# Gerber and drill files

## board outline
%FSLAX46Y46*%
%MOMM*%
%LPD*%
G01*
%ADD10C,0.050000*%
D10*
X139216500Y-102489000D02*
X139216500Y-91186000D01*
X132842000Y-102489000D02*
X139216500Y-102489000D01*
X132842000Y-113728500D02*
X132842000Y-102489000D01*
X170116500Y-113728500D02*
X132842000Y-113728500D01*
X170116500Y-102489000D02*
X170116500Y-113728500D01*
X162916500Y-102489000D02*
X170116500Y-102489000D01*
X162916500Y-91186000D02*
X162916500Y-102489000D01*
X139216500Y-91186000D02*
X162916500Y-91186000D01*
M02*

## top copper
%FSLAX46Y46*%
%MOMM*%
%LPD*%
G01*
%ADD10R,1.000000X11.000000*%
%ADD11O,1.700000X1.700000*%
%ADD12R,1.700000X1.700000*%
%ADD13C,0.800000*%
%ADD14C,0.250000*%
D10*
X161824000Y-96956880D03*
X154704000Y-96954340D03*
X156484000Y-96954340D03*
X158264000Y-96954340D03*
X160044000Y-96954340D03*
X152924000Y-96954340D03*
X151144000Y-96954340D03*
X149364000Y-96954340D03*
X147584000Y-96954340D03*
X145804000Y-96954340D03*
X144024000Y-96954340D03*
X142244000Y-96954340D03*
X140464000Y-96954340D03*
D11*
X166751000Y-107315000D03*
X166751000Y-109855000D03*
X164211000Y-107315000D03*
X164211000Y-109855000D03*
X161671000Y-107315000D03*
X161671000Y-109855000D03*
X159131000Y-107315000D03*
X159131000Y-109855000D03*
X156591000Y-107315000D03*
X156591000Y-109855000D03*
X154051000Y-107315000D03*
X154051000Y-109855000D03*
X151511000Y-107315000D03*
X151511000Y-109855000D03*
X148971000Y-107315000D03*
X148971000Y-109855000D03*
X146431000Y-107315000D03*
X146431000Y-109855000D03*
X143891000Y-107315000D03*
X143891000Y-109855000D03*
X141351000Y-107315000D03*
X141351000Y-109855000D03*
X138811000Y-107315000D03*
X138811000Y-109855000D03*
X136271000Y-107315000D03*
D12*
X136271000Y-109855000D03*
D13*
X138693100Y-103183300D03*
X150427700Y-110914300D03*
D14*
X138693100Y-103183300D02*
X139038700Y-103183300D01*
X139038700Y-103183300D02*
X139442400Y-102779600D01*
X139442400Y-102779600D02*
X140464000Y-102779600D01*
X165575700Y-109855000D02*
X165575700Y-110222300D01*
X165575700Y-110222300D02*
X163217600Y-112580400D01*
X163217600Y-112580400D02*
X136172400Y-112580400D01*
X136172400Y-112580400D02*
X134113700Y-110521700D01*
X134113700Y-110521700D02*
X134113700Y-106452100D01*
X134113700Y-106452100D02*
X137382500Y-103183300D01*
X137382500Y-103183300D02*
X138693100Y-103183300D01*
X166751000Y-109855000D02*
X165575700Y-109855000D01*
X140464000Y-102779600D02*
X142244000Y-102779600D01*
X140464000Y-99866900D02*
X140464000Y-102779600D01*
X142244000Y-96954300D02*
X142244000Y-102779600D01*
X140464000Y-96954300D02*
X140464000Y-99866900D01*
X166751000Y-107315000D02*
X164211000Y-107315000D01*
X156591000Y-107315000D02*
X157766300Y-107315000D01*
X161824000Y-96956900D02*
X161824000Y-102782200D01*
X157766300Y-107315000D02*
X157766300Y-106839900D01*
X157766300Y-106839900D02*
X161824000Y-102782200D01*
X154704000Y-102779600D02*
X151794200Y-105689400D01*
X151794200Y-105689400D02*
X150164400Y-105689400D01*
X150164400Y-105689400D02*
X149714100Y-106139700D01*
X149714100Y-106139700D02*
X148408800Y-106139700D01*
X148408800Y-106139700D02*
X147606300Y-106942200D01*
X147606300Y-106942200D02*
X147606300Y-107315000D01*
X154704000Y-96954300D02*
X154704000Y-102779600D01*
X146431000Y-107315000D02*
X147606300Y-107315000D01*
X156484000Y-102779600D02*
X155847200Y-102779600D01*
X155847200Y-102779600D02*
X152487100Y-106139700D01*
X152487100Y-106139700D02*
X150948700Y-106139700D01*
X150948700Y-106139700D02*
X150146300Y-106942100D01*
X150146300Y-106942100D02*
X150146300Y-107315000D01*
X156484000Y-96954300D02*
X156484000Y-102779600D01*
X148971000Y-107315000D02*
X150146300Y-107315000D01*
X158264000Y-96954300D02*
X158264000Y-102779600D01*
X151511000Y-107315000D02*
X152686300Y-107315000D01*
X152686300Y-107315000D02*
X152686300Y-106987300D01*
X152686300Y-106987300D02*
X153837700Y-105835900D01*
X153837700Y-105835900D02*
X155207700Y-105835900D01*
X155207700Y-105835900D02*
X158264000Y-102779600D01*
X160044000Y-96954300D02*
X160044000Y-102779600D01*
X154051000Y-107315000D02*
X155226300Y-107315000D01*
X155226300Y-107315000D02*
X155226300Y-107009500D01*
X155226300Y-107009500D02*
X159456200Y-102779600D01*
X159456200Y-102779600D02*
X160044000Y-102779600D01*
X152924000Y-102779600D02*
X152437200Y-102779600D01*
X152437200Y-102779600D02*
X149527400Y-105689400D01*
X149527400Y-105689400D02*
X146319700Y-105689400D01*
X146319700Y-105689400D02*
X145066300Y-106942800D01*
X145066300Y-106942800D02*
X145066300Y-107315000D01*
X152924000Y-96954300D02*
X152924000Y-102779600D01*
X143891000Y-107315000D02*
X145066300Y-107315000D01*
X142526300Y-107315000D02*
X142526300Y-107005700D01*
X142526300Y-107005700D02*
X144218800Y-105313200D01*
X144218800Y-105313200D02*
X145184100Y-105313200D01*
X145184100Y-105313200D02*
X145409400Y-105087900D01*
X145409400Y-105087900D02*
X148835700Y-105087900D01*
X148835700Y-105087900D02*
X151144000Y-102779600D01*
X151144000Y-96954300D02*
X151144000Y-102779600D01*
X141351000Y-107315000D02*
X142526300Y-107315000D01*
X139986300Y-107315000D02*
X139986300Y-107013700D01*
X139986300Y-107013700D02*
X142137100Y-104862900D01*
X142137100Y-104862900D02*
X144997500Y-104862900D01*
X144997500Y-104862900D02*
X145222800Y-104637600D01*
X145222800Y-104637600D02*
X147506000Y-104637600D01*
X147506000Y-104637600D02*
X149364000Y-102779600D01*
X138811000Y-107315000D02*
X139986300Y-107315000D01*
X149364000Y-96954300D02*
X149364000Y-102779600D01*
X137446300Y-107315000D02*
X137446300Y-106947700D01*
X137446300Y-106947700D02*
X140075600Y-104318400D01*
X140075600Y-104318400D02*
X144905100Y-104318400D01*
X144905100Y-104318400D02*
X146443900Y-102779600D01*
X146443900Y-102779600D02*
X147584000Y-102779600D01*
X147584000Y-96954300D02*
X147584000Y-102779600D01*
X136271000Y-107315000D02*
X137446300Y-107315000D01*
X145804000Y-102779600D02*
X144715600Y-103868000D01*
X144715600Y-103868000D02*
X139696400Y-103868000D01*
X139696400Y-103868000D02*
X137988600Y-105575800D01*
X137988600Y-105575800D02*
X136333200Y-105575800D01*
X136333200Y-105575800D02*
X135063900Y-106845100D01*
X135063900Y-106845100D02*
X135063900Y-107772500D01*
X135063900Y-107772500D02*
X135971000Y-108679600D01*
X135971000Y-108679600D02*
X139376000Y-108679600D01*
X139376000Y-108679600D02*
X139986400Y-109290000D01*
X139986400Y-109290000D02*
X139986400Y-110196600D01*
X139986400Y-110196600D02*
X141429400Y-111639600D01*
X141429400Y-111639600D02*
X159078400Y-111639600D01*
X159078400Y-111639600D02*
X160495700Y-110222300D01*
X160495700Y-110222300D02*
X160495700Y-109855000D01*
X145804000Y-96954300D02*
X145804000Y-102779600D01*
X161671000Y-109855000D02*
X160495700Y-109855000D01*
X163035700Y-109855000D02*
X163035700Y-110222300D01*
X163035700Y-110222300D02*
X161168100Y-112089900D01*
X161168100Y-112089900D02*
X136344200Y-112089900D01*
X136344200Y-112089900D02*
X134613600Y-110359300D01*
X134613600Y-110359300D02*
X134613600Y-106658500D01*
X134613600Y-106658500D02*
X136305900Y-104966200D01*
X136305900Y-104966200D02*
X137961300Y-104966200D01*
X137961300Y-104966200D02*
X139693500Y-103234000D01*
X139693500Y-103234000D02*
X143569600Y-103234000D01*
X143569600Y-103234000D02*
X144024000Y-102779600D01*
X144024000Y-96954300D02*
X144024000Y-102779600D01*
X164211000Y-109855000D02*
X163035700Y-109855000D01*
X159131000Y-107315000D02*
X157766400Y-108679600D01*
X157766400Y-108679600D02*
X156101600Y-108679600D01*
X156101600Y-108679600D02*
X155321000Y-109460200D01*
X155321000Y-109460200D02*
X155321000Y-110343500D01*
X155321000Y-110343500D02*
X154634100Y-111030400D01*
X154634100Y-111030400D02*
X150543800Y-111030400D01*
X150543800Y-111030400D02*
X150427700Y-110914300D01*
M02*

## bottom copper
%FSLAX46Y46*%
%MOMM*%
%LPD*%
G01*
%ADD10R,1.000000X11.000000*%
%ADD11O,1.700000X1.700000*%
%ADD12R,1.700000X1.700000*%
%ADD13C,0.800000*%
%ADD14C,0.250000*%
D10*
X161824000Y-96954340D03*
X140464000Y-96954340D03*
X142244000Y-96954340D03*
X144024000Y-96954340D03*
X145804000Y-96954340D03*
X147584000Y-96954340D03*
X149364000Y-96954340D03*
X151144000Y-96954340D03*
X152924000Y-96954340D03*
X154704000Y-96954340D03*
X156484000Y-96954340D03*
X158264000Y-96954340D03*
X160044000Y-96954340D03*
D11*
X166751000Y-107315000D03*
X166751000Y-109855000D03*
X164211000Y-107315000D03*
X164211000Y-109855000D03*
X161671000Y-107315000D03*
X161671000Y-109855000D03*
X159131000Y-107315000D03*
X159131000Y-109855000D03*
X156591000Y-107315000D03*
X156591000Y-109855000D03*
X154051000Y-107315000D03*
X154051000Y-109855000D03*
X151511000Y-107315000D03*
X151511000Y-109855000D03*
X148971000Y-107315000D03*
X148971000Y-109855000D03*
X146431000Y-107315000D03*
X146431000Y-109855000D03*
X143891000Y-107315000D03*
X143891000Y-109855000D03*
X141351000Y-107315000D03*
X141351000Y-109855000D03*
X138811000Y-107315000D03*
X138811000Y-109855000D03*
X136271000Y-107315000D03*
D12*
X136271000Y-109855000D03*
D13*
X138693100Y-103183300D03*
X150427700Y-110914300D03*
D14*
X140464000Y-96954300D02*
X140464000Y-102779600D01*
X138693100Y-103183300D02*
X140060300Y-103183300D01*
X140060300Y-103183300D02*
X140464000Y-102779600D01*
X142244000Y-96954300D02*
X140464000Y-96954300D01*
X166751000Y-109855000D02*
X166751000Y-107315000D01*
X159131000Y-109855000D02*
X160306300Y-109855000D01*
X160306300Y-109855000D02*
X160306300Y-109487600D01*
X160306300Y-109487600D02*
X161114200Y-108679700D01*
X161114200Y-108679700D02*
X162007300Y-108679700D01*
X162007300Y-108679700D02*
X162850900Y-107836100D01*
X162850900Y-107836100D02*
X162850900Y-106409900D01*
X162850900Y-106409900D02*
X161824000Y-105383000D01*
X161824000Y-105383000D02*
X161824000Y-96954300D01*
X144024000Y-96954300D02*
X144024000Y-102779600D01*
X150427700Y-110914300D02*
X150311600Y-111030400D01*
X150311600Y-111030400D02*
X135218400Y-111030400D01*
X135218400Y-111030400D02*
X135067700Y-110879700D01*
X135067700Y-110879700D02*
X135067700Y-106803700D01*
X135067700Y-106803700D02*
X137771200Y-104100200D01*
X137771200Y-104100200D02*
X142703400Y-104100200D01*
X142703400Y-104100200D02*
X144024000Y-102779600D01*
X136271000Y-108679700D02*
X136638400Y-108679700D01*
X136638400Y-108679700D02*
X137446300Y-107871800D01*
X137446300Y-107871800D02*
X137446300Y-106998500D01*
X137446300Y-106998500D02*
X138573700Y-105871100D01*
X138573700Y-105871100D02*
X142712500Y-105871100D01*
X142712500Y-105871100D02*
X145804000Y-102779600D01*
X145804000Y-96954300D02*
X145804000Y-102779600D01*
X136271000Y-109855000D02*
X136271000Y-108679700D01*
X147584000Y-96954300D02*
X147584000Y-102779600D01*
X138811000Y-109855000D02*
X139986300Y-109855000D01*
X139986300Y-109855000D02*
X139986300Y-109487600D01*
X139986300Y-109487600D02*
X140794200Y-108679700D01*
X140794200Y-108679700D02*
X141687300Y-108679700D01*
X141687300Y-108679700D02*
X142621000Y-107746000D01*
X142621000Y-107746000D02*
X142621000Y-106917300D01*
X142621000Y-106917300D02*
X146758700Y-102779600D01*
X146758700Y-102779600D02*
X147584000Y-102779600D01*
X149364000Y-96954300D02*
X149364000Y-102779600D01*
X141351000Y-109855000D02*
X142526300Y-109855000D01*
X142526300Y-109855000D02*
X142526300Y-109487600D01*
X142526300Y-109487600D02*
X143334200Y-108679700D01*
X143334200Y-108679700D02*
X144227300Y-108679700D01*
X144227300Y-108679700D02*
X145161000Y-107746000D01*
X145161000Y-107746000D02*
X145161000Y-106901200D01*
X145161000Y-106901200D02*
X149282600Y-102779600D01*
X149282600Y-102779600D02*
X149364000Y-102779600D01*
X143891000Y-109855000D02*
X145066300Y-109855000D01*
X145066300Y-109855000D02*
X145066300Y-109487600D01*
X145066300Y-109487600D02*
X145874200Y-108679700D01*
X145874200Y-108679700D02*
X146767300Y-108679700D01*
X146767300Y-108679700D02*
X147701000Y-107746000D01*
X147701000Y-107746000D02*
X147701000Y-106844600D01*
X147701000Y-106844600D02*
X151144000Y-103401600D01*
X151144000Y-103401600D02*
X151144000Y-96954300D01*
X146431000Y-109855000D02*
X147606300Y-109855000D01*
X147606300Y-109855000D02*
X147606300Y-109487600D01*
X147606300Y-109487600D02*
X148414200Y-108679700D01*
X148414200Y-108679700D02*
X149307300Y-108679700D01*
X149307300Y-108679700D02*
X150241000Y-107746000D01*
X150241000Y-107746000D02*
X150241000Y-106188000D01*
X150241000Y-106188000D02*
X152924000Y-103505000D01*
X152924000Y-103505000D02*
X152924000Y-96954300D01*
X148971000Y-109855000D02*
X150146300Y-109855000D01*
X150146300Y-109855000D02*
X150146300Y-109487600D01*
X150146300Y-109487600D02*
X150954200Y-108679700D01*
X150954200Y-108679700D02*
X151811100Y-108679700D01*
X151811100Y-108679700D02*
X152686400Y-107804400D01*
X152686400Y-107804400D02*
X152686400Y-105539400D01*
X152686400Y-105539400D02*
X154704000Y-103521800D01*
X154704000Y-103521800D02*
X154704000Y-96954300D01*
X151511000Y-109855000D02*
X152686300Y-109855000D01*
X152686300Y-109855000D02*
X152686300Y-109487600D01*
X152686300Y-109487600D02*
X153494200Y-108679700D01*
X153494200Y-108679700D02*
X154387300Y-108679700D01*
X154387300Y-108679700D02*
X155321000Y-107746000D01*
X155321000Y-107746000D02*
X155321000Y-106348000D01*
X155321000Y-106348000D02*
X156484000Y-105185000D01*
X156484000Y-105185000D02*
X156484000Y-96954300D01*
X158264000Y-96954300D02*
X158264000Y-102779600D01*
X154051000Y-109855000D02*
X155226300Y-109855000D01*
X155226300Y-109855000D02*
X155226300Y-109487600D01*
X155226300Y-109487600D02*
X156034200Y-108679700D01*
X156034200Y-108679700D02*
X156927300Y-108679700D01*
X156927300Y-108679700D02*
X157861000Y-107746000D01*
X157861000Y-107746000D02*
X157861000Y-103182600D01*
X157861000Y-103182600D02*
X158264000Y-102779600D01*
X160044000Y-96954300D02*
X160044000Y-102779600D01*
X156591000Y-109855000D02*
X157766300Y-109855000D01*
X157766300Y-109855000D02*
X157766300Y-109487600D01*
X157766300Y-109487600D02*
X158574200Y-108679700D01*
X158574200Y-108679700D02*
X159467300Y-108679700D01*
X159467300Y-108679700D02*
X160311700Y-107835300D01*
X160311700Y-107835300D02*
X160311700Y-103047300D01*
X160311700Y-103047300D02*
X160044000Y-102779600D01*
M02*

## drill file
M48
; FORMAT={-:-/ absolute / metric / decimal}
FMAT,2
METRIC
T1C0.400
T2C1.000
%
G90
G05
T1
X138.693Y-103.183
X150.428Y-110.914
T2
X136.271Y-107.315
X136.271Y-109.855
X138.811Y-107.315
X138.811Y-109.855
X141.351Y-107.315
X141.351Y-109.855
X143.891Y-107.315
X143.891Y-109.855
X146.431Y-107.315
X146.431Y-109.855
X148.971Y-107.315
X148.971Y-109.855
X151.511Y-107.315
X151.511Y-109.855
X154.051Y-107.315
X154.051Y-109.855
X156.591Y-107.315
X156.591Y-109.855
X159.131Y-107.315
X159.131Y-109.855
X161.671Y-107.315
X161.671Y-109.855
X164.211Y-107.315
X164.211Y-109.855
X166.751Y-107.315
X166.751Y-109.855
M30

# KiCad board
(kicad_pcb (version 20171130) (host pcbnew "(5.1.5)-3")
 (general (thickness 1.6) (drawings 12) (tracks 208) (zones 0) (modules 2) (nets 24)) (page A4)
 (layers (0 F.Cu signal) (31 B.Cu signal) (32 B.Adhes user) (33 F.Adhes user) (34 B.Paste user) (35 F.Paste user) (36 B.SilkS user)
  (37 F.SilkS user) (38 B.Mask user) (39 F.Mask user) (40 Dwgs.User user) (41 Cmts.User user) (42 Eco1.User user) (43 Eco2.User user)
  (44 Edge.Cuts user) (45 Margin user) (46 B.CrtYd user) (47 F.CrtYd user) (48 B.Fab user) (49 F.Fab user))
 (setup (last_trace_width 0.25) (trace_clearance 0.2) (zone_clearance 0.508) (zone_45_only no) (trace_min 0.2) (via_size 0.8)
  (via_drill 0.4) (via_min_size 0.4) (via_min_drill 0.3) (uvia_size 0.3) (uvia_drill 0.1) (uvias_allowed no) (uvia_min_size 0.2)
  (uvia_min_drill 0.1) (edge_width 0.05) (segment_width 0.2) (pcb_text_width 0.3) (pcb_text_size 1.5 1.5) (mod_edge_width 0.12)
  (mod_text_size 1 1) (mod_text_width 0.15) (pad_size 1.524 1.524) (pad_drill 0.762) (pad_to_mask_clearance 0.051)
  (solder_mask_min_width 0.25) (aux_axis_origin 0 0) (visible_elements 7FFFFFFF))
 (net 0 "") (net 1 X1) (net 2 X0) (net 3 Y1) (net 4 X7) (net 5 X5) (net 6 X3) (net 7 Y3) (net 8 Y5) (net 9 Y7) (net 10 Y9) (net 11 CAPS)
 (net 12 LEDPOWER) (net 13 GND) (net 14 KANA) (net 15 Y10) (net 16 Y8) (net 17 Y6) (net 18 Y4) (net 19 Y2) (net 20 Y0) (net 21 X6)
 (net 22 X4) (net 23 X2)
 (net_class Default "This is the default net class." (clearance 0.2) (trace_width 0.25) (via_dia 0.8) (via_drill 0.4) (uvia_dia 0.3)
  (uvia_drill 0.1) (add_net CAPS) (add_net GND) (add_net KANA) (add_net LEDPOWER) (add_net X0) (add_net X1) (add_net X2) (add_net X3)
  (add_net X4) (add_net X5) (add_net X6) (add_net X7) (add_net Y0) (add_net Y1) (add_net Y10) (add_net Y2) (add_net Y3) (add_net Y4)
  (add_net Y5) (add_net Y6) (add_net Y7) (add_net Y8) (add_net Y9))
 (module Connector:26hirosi (layer F.Cu) (at 152.464 97.028)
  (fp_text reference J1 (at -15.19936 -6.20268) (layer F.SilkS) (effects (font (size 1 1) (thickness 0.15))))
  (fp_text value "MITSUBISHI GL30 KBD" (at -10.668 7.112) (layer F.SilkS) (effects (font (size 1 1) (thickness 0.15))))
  (pad 25 connect rect (at 9.36 -0.07112) (size 1 11) (layers F.Cu F.Mask) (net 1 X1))
  (pad 26 connect rect (at 9.36 -0.07366) (size 1 11) (layers B.Cu B.Mask) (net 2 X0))
  (pad 17 connect rect (at 2.24 -0.07366) (size 1 11) (layers F.Cu F.Mask) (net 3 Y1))
  (pad 19 connect rect (at 4.02 -0.07366) (size 1 11) (layers F.Cu F.Mask) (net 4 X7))
  (pad 21 connect rect (at 5.8 -0.07366) (size 1 11) (layers F.Cu F.Mask) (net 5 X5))
  (pad 23 connect rect (at 7.58 -0.07366) (size 1 11) (layers F.Cu F.Mask) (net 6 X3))
  (pad 15 connect rect (at 0.46 -0.07366) (size 1 11) (layers F.Cu F.Mask) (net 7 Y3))
  (pad 13 connect rect (at -1.32 -0.07366) (size 1 11) (layers F.Cu F.Mask) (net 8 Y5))
  (pad 11 connect rect (at -3.1 -0.07366) (size 1 11) (layers F.Cu F.Mask) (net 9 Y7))
  (pad 9 connect rect (at -4.88 -0.07366) (size 1 11) (layers F.Cu F.Mask) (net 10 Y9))
  (pad 7 connect rect (at -6.66 -0.07366) (size 1 11) (layers F.Cu F.Mask) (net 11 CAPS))
  (pad 5 connect rect (at -8.44 -0.07366) (size 1 11) (layers F.Cu F.Mask) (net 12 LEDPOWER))
  (pad 3 connect rect (at -10.22 -0.07366) (size 1 11) (layers F.Cu F.Mask) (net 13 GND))
  (pad 1 connect rect (at -12 -0.07366) (size 1 11) (layers F.Cu F.Mask) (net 13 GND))
  (pad 2 connect rect (at -12 -0.07366) (size 1 11) (layers B.Cu B.Mask) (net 13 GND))
  (pad 4 connect rect (at -10.22 -0.07366) (size 1 11) (layers B.Cu B.Mask) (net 13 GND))
  (pad 6 connect rect (at -8.44 -0.07366) (size 1 11) (layers B.Cu B.Mask) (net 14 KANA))
  (pad 8 connect rect (at -6.66 -0.07366) (size 1 11) (layers B.Cu B.Mask) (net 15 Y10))
  (pad 10 connect rect (at -4.88 -0.07366) (size 1 11) (layers B.Cu B.Mask) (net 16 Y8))
  (pad 12 connect rect (at -3.1 -0.07366) (size 1 11) (layers B.Cu B.Mask) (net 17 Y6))
  (pad 14 connect rect (at -1.32 -0.07366) (size 1 11) (layers B.Cu B.Mask) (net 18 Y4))
  (pad 16 connect rect (at 0.46 -0.07366) (size 1 11) (layers B.Cu B.Mask) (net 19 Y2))
  (pad 18 connect rect (at 2.24 -0.07366) (size 1 11) (layers B.Cu B.Mask) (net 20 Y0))
  (pad 20 connect rect (at 4.02 -0.07366) (size 1 11) (layers B.Cu B.Mask) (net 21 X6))
  (pad 22 connect rect (at 5.8 -0.07366) (size 1 11) (layers B.Cu B.Mask) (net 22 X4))
  (pad 24 connect rect (at 7.58 -0.07366) (size 1 11) (layers B.Cu B.Mask) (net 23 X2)))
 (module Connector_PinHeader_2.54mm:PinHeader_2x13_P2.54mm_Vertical (layer F.Cu) (at 136.271 109.855 90)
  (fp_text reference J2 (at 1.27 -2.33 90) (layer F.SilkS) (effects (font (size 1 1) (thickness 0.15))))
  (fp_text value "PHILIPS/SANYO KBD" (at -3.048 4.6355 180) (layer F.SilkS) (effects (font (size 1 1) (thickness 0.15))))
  (pad 26 thru_hole oval (at 2.54 30.48 90) (size 1.7 1.7) (drill 1) (layers *.Cu *.Mask) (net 13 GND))
  (pad 25 thru_hole oval (at 0 30.48 90) (size 1.7 1.7) (drill 1) (layers *.Cu *.Mask) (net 13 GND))
  (pad 24 thru_hole oval (at 2.54 27.94 90) (size 1.7 1.7) (drill 1) (layers *.Cu *.Mask) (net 13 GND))
  (pad 23 thru_hole oval (at 0 27.94 90) (size 1.7 1.7) (drill 1) (layers *.Cu *.Mask) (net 12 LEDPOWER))
  (pad 22 thru_hole oval (at 2.54 25.4 90) (size 1.7 1.7) (drill 1) (layers *.Cu *.Mask))
  (pad 21 thru_hole oval (at 0 25.4 90) (size 1.7 1.7) (drill 1) (layers *.Cu *.Mask) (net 11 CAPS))
  (pad 20 thru_hole oval (at 2.54 22.86 90) (size 1.7 1.7) (drill 1) (layers *.Cu *.Mask) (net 14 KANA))
  (pad 19 thru_hole oval (at 0 22.86 90) (size 1.7 1.7) (drill 1) (layers *.Cu *.Mask) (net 2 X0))
  (pad 18 thru_hole oval (at 2.54 20.32 90) (size 1.7 1.7) (drill 1) (layers *.Cu *.Mask) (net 1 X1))
  (pad 17 thru_hole oval (at 0 20.32 90) (size 1.7 1.7) (drill 1) (layers *.Cu *.Mask) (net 23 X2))
  (pad 16 thru_hole oval (at 2.54 17.78 90) (size 1.7 1.7) (drill 1) (layers *.Cu *.Mask) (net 6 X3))
  (pad 15 thru_hole oval (at 0 17.78 90) (size 1.7 1.7) (drill 1) (layers *.Cu *.Mask) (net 22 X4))
  (pad 14 thru_hole oval (at 2.54 15.24 90) (size 1.7 1.7) (drill 1) (layers *.Cu *.Mask) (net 5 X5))
  (pad 13 thru_hole oval (at 0 15.24 90) (size 1.7 1.7) (drill 1) (layers *.Cu *.Mask) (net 21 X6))
  (pad 12 thru_hole oval (at 2.54 12.7 90) (size 1.7 1.7) (drill 1) (layers *.Cu *.Mask) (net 4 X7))
  (pad 11 thru_hole oval (at 0 12.7 90) (size 1.7 1.7) (drill 1) (layers *.Cu *.Mask) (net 20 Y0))
  (pad 10 thru_hole oval (at 2.54 10.16 90) (size 1.7 1.7) (drill 1) (layers *.Cu *.Mask) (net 3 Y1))
  (pad 9 thru_hole oval (at 0 10.16 90) (size 1.7 1.7) (drill 1) (layers *.Cu *.Mask) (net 19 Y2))
  (pad 8 thru_hole oval (at 2.54 7.62 90) (size 1.7 1.7) (drill 1) (layers *.Cu *.Mask) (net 7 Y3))
  (pad 7 thru_hole oval (at 0 7.62 90) (size 1.7 1.7) (drill 1) (layers *.Cu *.Mask) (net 18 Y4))
  (pad 6 thru_hole oval (at 2.54 5.08 90) (size 1.7 1.7) (drill 1) (layers *.Cu *.Mask) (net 8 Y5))
  (pad 5 thru_hole oval (at 0 5.08 90) (size 1.7 1.7) (drill 1) (layers *.Cu *.Mask) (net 17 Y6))
  (pad 4 thru_hole oval (at 2.54 2.54 90) (size 1.7 1.7) (drill 1) (layers *.Cu *.Mask) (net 9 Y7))
  (pad 3 thru_hole oval (at 0 2.54 90) (size 1.7 1.7) (drill 1) (layers *.Cu *.Mask) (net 16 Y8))
  (pad 2 thru_hole oval (at 2.54 0 90) (size 1.7 1.7) (drill 1) (layers *.Cu *.Mask) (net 10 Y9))
  (pad 1 thru_hole rect (at 0 0 90) (size 1.7 1.7) (drill 1) (layers *.Cu *.Mask) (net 15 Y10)))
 (gr_line (start 139.2165 102.489) (end 139.2165 91.186) (layer Edge.Cuts) (width 0.05))
 (gr_line (start 132.842 102.489) (end 139.2165 102.489) (layer Edge.Cuts) (width 0.05))
 (gr_line (start 132.842 113.7285) (end 132.842 102.489) (layer Edge.Cuts) (width 0.05))
 (gr_line (start 170.1165 113.7285) (end 132.842 113.7285) (layer Edge.Cuts) (width 0.05))
 (gr_line (start 170.1165 102.489) (end 170.1165 113.7285) (layer Edge.Cuts) (width 0.05))
 (gr_line (start 162.9165 102.489) (end 170.1165 102.489) (layer Edge.Cuts) (width 0.05))
 (gr_line (start 162.9165 91.186) (end 162.9165 102.489) (layer Edge.Cuts) (width 0.05))
 (gr_line (start 139.2165 91.186) (end 162.9165 91.186) (layer Edge.Cuts) (width 0.05))
 (segment (start 138.6931 103.1833) (end 139.0387 103.1833) (width 0.25) (layer F.Cu) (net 13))
 (segment (start 139.0387 103.1833) (end 139.4424 102.7796) (width 0.25) (layer F.Cu) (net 13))
 (segment (start 139.4424 102.7796) (end 140.464 102.7796) (width 0.25) (layer F.Cu) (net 13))
 (segment (start 165.5757 109.855) (end 165.5757 110.2223) (width 0.25) (layer F.Cu) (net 13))
 (segment (start 165.5757 110.2223) (end 163.2176 112.5804) (width 0.25) (layer F.Cu) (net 13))
 (segment (start 163.2176 112.5804) (end 136.1724 112.5804) (width 0.25) (layer F.Cu) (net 13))
 (segment (start 136.1724 112.5804) (end 134.1137 110.5217) (width 0.25) (layer F.Cu) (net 13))
 (segment (start 134.1137 110.5217) (end 134.1137 106.4521) (width 0.25) (layer F.Cu) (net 13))
 (segment (start 134.1137 106.4521) (end 137.3825 103.1833) (width 0.25) (layer F.Cu) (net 13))
 (segment (start 137.3825 103.1833) (end 138.6931 103.1833) (width 0.25) (layer F.Cu) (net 13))
 (segment (start 140.464 96.9543) (end 140.464 102.7796) (width 0.25) (layer B.Cu) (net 13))
 (segment (start 138.6931 103.1833) (end 140.0603 103.1833) (width 0.25) (layer B.Cu) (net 13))
 (segment (start 140.0603 103.1833) (end 140.464 102.7796) (width 0.25) (layer B.Cu) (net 13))
 (segment (start 142.244 96.9543) (end 140.464 96.9543) (width 0.25) (layer B.Cu) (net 13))
 (segment (start 166.751 109.855) (end 165.5757 109.855) (width 0.25) (layer F.Cu) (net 13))
 (segment (start 140.464 102.7796) (end 142.244 102.7796) (width 0.25) (layer F.Cu) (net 13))
 (segment (start 140.464 99.8669) (end 140.464 102.7796) (width 0.25) (layer F.Cu) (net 13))
 (segment (start 166.751 109.855) (end 166.751 107.315) (width 0.25) (layer B.Cu) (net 13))
 (segment (start 142.244 96.9543) (end 142.244 102.7796) (width 0.25) (layer F.Cu) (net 13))
 (segment (start 140.464 96.9543) (end 140.464 99.8669) (width 0.25) (layer F.Cu) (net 13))
 (segment (start 166.751 107.315) (end 164.211 107.315) (width 0.25) (layer F.Cu) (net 13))
 (via (at 138.6931 103.1833) (size 0.8) (layers F.Cu B.Cu) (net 13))
 (segment (start 156.591 107.315) (end 157.7663 107.315) (width 0.25) (layer F.Cu) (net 1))
 (segment (start 161.824 96.9569) (end 161.824 102.7822) (width 0.25) (layer F.Cu) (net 1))
 (segment (start 157.7663 107.315) (end 157.7663 106.8399) (width 0.25) (layer F.Cu) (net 1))
 (segment (start 157.7663 106.8399) (end 161.824 102.7822) (width 0.25) (layer F.Cu) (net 1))
 (segment (start 159.131 109.855) (end 160.3063 109.855) (width 0.25) (layer B.Cu) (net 2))
 (segment (start 160.3063 109.855) (end 160.3063 109.4876) (width 0.25) (layer B.Cu) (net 2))
 (segment (start 160.3063 109.4876) (end 161.1142 108.6797) (width 0.25) (layer B.Cu) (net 2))
 (segment (start 161.1142 108.6797) (end 162.0073 108.6797) (width 0.25) (layer B.Cu) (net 2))
 (segment (start 162.0073 108.6797) (end 162.8509 107.8361) (width 0.25) (layer B.Cu) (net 2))
 (segment (start 162.8509 107.8361) (end 162.8509 106.4099) (width 0.25) (layer B.Cu) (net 2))
 (segment (start 162.8509 106.4099) (end 161.824 105.383) (width 0.25) (layer B.Cu) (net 2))
 (segment (start 161.824 105.383) (end 161.824 96.9543) (width 0.25) (layer B.Cu) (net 2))
 (segment (start 154.704 102.7796) (end 151.7942 105.6894) (width 0.25) (layer F.Cu) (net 3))
 (segment (start 151.7942 105.6894) (end 150.1644 105.6894) (width 0.25) (layer F.Cu) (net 3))
 (segment (start 150.1644 105.6894) (end 149.7141 106.1397) (width 0.25) (layer F.Cu) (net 3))
 (segment (start 149.7141 106.1397) (end 148.4088 106.1397) (width 0.25) (layer F.Cu) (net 3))
 (segment (start 148.4088 106.1397) (end 147.6063 106.9422) (width 0.25) (layer F.Cu) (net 3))
 (segment (start 147.6063 106.9422) (end 147.6063 107.315) (width 0.25) (layer F.Cu) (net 3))
 (segment (start 154.704 96.9543) (end 154.704 102.7796) (width 0.25) (layer F.Cu) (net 3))
 (segment (start 146.431 107.315) (end 147.6063 107.315) (width 0.25) (layer F.Cu) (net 3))
 (segment (start 156.484 102.7796) (end 155.8472 102.7796) (width 0.25) (layer F.Cu) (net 4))
 (segment (start 155.8472 102.7796) (end 152.4871 106.1397) (width 0.25) (layer F.Cu) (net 4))
 (segment (start 152.4871 106.1397) (end 150.9487 106.1397) (width 0.25) (layer F.Cu) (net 4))
 (segment (start 150.9487 106.1397) (end 150.1463 106.9421) (width 0.25) (layer F.Cu) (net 4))
 (segment (start 150.1463 106.9421) (end 150.1463 107.315) (width 0.25) (layer F.Cu) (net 4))
 (segment (start 156.484 96.9543) (end 156.484 102.7796) (width 0.25) (layer F.Cu) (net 4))
 (segment (start 148.971 107.315) (end 150.1463 107.315) (width 0.25) (layer F.Cu) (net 4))
 (segment (start 158.264 96.9543) (end 158.264 102.7796) (width 0.25) (layer F.Cu) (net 5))
 (segment (start 151.511 107.315) (end 152.6863 107.315) (width 0.25) (layer F.Cu) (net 5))
 (segment (start 152.6863 107.315) (end 152.6863 106.9873) (width 0.25) (layer F.Cu) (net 5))
 (segment (start 152.6863 106.9873) (end 153.8377 105.8359) (width 0.25) (layer F.Cu) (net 5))
 (segment (start 153.8377 105.8359) (end 155.2077 105.8359) (width 0.25) (layer F.Cu) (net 5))
 (segment (start 155.2077 105.8359) (end 158.264 102.7796) (width 0.25) (layer F.Cu) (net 5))
 (segment (start 160.044 96.9543) (end 160.044 102.7796) (width 0.25) (layer F.Cu) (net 6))
 (segment (start 154.051 107.315) (end 155.2263 107.315) (width 0.25) (layer F.Cu) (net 6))
 (segment (start 155.2263 107.315) (end 155.2263 107.0095) (width 0.25) (layer F.Cu) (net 6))
 (segment (start 155.2263 107.0095) (end 159.4562 102.7796) (width 0.25) (layer F.Cu) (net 6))
 (segment (start 159.4562 102.7796) (end 160.044 102.7796) (width 0.25) (layer F.Cu) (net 6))
 (segment (start 152.924 102.7796) (end 152.4372 102.7796) (width 0.25) (layer F.Cu) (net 7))
 (segment (start 152.4372 102.7796) (end 149.5274 105.6894) (width 0.25) (layer F.Cu) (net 7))
 (segment (start 149.5274 105.6894) (end 146.3197 105.6894) (width 0.25) (layer F.Cu) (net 7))
 (segment (start 146.3197 105.6894) (end 145.0663 106.9428) (width 0.25) (layer F.Cu) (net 7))
 (segment (start 145.0663 106.9428) (end 145.0663 107.315) (width 0.25) (layer F.Cu) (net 7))
 (segment (start 152.924 96.9543) (end 152.924 102.7796) (width 0.25) (layer F.Cu) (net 7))
 (segment (start 143.891 107.315) (end 145.0663 107.315) (width 0.25) (layer F.Cu) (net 7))
 (segment (start 142.5263 107.315) (end 142.5263 107.0057) (width 0.25) (layer F.Cu) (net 8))
 (segment (start 142.5263 107.0057) (end 144.2188 105.3132) (width 0.25) (layer F.Cu) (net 8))
 (segment (start 144.2188 105.3132) (end 145.1841 105.3132) (width 0.25) (layer F.Cu) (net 8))
 (segment (start 145.1841 105.3132) (end 145.4094 105.0879) (width 0.25) (layer F.Cu) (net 8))
 (segment (start 145.4094 105.0879) (end 148.8357 105.0879) (width 0.25) (layer F.Cu) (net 8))
 (segment (start 148.8357 105.0879) (end 151.144 102.7796) (width 0.25) (layer F.Cu) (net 8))
 (segment (start 151.144 96.9543) (end 151.144 102.7796) (width 0.25) (layer F.Cu) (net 8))
 (segment (start 141.351 107.315) (end 142.5263 107.315) (width 0.25) (layer F.Cu) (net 8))
 (segment (start 139.9863 107.315) (end 139.9863 107.0137) (width 0.25) (layer F.Cu) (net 9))
 (segment (start 139.9863 107.0137) (end 142.1371 104.8629) (width 0.25) (layer F.Cu) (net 9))
 (segment (start 142.1371 104.8629) (end 144.9975 104.8629) (width 0.25) (layer F.Cu) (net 9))
 (segment (start 144.9975 104.8629) (end 145.2228 104.6376) (width 0.25) (layer F.Cu) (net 9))
 (segment (start 145.2228 104.6376) (end 147.506 104.6376) (width 0.25) (layer F.Cu) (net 9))
 (segment (start 147.506 104.6376) (end 149.364 102.7796) (width 0.25) (layer F.Cu) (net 9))
 (segment (start 138.811 107.315) (end 139.9863 107.315) (width 0.25) (layer F.Cu) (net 9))
 (segment (start 149.364 96.9543) (end 149.364 102.7796) (width 0.25) (layer F.Cu) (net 9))
 (segment (start 137.4463 107.315) (end 137.4463 106.9477) (width 0.25) (layer F.Cu) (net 10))
 (segment (start 137.4463 106.9477) (end 140.0756 104.3184) (width 0.25) (layer F.Cu) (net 10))
 (segment (start 140.0756 104.3184) (end 144.9051 104.3184) (width 0.25) (layer F.Cu) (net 10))
 (segment (start 144.9051 104.3184) (end 146.4439 102.7796) (width 0.25) (layer F.Cu) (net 10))
 (segment (start 146.4439 102.7796) (end 147.584 102.7796) (width 0.25) (layer F.Cu) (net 10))
 (segment (start 147.584 96.9543) (end 147.584 102.7796) (width 0.25) (layer F.Cu) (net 10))
 (segment (start 136.271 107.315) (end 137.4463 107.315) (width 0.25) (layer F.Cu) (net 10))
 (segment (start 145.804 102.7796) (end 144.7156 103.868) (width 0.25) (layer F.Cu) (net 11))
 (segment (start 144.7156 103.868) (end 139.6964 103.868) (width 0.25) (layer F.Cu) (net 11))
 (segment (start 139.6964 103.868) (end 137.9886 105.5758) (width 0.25) (layer F.Cu) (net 11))
 (segment (start 137.9886 105.5758) (end 136.3332 105.5758) (width 0.25) (layer F.Cu) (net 11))
 (segment (start 136.3332 105.5758) (end 135.0639 106.8451) (width 0.25) (layer F.Cu) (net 11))
 (segment (start 135.0639 106.8451) (end 135.0639 107.7725) (width 0.25) (layer F.Cu) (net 11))
 (segment (start 135.0639 107.7725) (end 135.971 108.6796) (width 0.25) (layer F.Cu) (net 11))
 (segment (start 135.971 108.6796) (end 139.376 108.6796) (width 0.25) (layer F.Cu) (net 11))
 (segment (start 139.376 108.6796) (end 139.9864 109.29) (width 0.25) (layer F.Cu) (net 11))
 (segment (start 139.9864 109.29) (end 139.9864 110.1966) (width 0.25) (layer F.Cu) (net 11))
 (segment (start 139.9864 110.1966) (end 141.4294 111.6396) (width 0.25) (layer F.Cu) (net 11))
 (segment (start 141.4294 111.6396) (end 159.0784 111.6396) (width 0.25) (layer F.Cu) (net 11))
 (segment (start 159.0784 111.6396) (end 160.4957 110.2223) (width 0.25) (layer F.Cu) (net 11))
 (segment (start 160.4957 110.2223) (end 160.4957 109.855) (width 0.25) (layer F.Cu) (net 11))
 (segment (start 145.804 96.9543) (end 145.804 102.7796) (width 0.25) (layer F.Cu) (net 11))
 (segment (start 161.671 109.855) (end 160.4957 109.855) (width 0.25) (layer F.Cu) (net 11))
 (segment (start 163.0357 109.855) (end 163.0357 110.2223) (width 0.25) (layer F.Cu) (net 12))
 (segment (start 163.0357 110.2223) (end 161.1681 112.0899) (width 0.25) (layer F.Cu) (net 12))
 (segment (start 161.1681 112.0899) (end 136.3442 112.0899) (width 0.25) (layer F.Cu) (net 12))
 (segment (start 136.3442 112.0899) (end 134.6136 110.3593) (width 0.25) (layer F.Cu) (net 12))
 (segment (start 134.6136 110.3593) (end 134.6136 106.6585) (width 0.25) (layer F.Cu) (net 12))
 (segment (start 134.6136 106.6585) (end 136.3059 104.9662) (width 0.25) (layer F.Cu) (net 12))
 (segment (start 136.3059 104.9662) (end 137.9613 104.9662) (width 0.25) (layer F.Cu) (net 12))
 (segment (start 137.9613 104.9662) (end 139.6935 103.234) (width 0.25) (layer F.Cu) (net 12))
 (segment (start 139.6935 103.234) (end 143.5696 103.234) (width 0.25) (layer F.Cu) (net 12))
 (segment (start 143.5696 103.234) (end 144.024 102.7796) (width 0.25) (layer F.Cu) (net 12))
 (segment (start 144.024 96.9543) (end 144.024 102.7796) (width 0.25) (layer F.Cu) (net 12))
 (segment (start 164.211 109.855) (end 163.0357 109.855) (width 0.25) (layer F.Cu) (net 12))
 (segment (start 144.024 96.9543) (end 144.024 102.7796) (width 0.25) (layer B.Cu) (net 14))
 (segment (start 150.4277 110.9143) (end 150.3116 111.0304) (width 0.25) (layer B.Cu) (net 14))
 (segment (start 150.3116 111.0304) (end 135.2184 111.0304) (width 0.25) (layer B.Cu) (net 14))
 (segment (start 135.2184 111.0304) (end 135.0677 110.8797) (width 0.25) (layer B.Cu) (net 14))
 (segment (start 135.0677 110.8797) (end 135.0677 106.8037) (width 0.25) (layer B.Cu) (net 14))
 (segment (start 135.0677 106.8037) (end 137.7712 104.1002) (width 0.25) (layer B.Cu) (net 14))
 (segment (start 137.7712 104.1002) (end 142.7034 104.1002) (width 0.25) (layer B.Cu) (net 14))
 (segment (start 142.7034 104.1002) (end 144.024 102.7796) (width 0.25) (layer B.Cu) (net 14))
 (segment (start 159.131 107.315) (end 157.7664 108.6796) (width 0.25) (layer F.Cu) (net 14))
 (segment (start 157.7664 108.6796) (end 156.1016 108.6796) (width 0.25) (layer F.Cu) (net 14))
 (segment (start 156.1016 108.6796) (end 155.321 109.4602) (width 0.25) (layer F.Cu) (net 14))
 (segment (start 155.321 109.4602) (end 155.321 110.3435) (width 0.25) (layer F.Cu) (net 14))
 (segment (start 155.321 110.3435) (end 154.6341 111.0304) (width 0.25) (layer F.Cu) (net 14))
 (segment (start 154.6341 111.0304) (end 150.5438 111.0304) (width 0.25) (layer F.Cu) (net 14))
 (segment (start 150.5438 111.0304) (end 150.4277 110.9143) (width 0.25) (layer F.Cu) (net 14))
 (via (at 150.4277 110.9143) (size 0.8) (layers F.Cu B.Cu) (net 14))
 (segment (start 136.271 108.6797) (end 136.6384 108.6797) (width 0.25) (layer B.Cu) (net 15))
 (segment (start 136.6384 108.6797) (end 137.4463 107.8718) (width 0.25) (layer B.Cu) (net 15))
 (segment (start 137.4463 107.8718) (end 137.4463 106.9985) (width 0.25) (layer B.Cu) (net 15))
 (segment (start 137.4463 106.9985) (end 138.5737 105.8711) (width 0.25) (layer B.Cu) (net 15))
 (segment (start 138.5737 105.8711) (end 142.7125 105.8711) (width 0.25) (layer B.Cu) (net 15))
 (segment (start 142.7125 105.8711) (end 145.804 102.7796) (width 0.25) (layer B.Cu) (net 15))
 (segment (start 145.804 96.9543) (end 145.804 102.7796) (width 0.25) (layer B.Cu) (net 15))
 (segment (start 136.271 109.855) (end 136.271 108.6797) (width 0.25) (layer B.Cu) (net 15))
 (segment (start 147.584 96.9543) (end 147.584 102.7796) (width 0.25) (layer B.Cu) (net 16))
 (segment (start 138.811 109.855) (end 139.9863 109.855) (width 0.25) (layer B.Cu) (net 16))
 (segment (start 139.9863 109.855) (end 139.9863 109.4876) (width 0.25) (layer B.Cu) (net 16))
 (segment (start 139.9863 109.4876) (end 140.7942 108.6797) (width 0.25) (layer B.Cu) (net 16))
 (segment (start 140.7942 108.6797) (end 141.6873 108.6797) (width 0.25) (layer B.Cu) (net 16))
 (segment (start 141.6873 108.6797) (end 142.621 107.746) (width 0.25) (layer B.Cu) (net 16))
 (segment (start 142.621 107.746) (end 142.621 106.9173) (width 0.25) (layer B.Cu) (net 16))
 (segment (start 142.621 106.9173) (end 146.7587 102.7796) (width 0.25) (layer B.Cu) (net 16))
 (segment (start 146.7587 102.7796) (end 147.584 102.7796) (width 0.25) (layer B.Cu) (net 16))
 (segment (start 149.364 96.9543) (end 149.364 102.7796) (width 0.25) (layer B.Cu) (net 17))
 (segment (start 141.351 109.855) (end 142.5263 109.855) (width 0.25) (layer B.Cu) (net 17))
 (segment (start 142.5263 109.855) (end 142.5263 109.4876) (width 0.25) (layer B.Cu) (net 17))
 (segment (start 142.5263 109.4876) (end 143.3342 108.6797) (width 0.25) (layer B.Cu) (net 17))
 (segment (start 143.3342 108.6797) (end 144.2273 108.6797) (width 0.25) (layer B.Cu) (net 17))
 (segment (start 144.2273 108.6797) (end 145.161 107.746) (width 0.25) (layer B.Cu) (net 17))
 (segment (start 145.161 107.746) (end 145.161 106.9012) (width 0.25) (layer B.Cu) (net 17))
 (segment (start 145.161 106.9012) (end 149.2826 102.7796) (width 0.25) (layer B.Cu) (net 17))
 (segment (start 149.2826 102.7796) (end 149.364 102.7796) (width 0.25) (layer B.Cu) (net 17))
 (segment (start 143.891 109.855) (end 145.0663 109.855) (width 0.25) (layer B.Cu) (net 18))
 (segment (start 145.0663 109.855) (end 145.0663 109.4876) (width 0.25) (layer B.Cu) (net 18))
 (segment (start 145.0663 109.4876) (end 145.8742 108.6797) (width 0.25) (layer B.Cu) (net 18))
 (segment (start 145.8742 108.6797) (end 146.7673 108.6797) (width 0.25) (layer B.Cu) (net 18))
 (segment (start 146.7673 108.6797) (end 147.701 107.746) (width 0.25) (layer B.Cu) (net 18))
 (segment (start 147.701 107.746) (end 147.701 106.8446) (width 0.25) (layer B.Cu) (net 18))
 (segment (start 147.701 106.8446) (end 151.144 103.4016) (width 0.25) (layer B.Cu) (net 18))
 (segment (start 151.144 103.4016) (end 151.144 96.9543) (width 0.25) (layer B.Cu) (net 18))
 (segment (start 146.431 109.855) (end 147.6063 109.855) (width 0.25) (layer B.Cu) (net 19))
 (segment (start 147.6063 109.855) (end 147.6063 109.4876) (width 0.25) (layer B.Cu) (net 19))
 (segment (start 147.6063 109.4876) (end 148.4142 108.6797) (width 0.25) (layer B.Cu) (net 19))
 (segment (start 148.4142 108.6797) (end 149.3073 108.6797) (width 0.25) (layer B.Cu) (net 19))
 (segment (start 149.3073 108.6797) (end 150.241 107.746) (width 0.25) (layer B.Cu) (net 19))
 (segment (start 150.241 107.746) (end 150.241 106.188) (width 0.25) (layer B.Cu) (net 19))
 (segment (start 150.241 106.188) (end 152.924 103.505) (width 0.25) (layer B.Cu) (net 19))
 (segment (start 152.924 103.505) (end 152.924 96.9543) (width 0.25) (layer B.Cu) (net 19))
 (segment (start 148.971 109.855) (end 150.1463 109.855) (width 0.25) (layer B.Cu) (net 20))
 (segment (start 150.1463 109.855) (end 150.1463 109.4876) (width 0.25) (layer B.Cu) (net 20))
 (segment (start 150.1463 109.4876) (end 150.9542 108.6797) (width 0.25) (layer B.Cu) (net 20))
 (segment (start 150.9542 108.6797) (end 151.8111 108.6797) (width 0.25) (layer B.Cu) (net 20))
 (segment (start 151.8111 108.6797) (end 152.6864 107.8044) (width 0.25) (layer B.Cu) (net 20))
 (segment (start 152.6864 107.8044) (end 152.6864 105.5394) (width 0.25) (layer B.Cu) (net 20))
 (segment (start 152.6864 105.5394) (end 154.704 103.5218) (width 0.25) (layer B.Cu) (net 20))
 (segment (start 154.704 103.5218) (end 154.704 96.9543) (width 0.25) (layer B.Cu) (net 20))
 (segment (start 151.511 109.855) (end 152.6863 109.855) (width 0.25) (layer B.Cu) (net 21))
 (segment (start 152.6863 109.855) (end 152.6863 109.4876) (width 0.25) (layer B.Cu) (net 21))
 (segment (start 152.6863 109.4876) (end 153.4942 108.6797) (width 0.25) (layer B.Cu) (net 21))
 (segment (start 153.4942 108.6797) (end 154.3873 108.6797) (width 0.25) (layer B.Cu) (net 21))
 (segment (start 154.3873 108.6797) (end 155.321 107.746) (width 0.25) (layer B.Cu) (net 21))
 (segment (start 155.321 107.746) (end 155.321 106.348) (width 0.25) (layer B.Cu) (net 21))
 (segment (start 155.321 106.348) (end 156.484 105.185) (width 0.25) (layer B.Cu) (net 21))
 (segment (start 156.484 105.185) (end 156.484 96.9543) (width 0.25) (layer B.Cu) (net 21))
 (segment (start 158.264 96.9543) (end 158.264 102.7796) (width 0.25) (layer B.Cu) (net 22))
 (segment (start 154.051 109.855) (end 155.2263 109.855) (width 0.25) (layer B.Cu) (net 22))
 (segment (start 155.2263 109.855) (end 155.2263 109.4876) (width 0.25) (layer B.Cu) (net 22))
 (segment (start 155.2263 109.4876) (end 156.0342 108.6797) (width 0.25) (layer B.Cu) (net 22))
 (segment (start 156.0342 108.6797) (end 156.9273 108.6797) (width 0.25) (layer B.Cu) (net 22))
 (segment (start 156.9273 108.6797) (end 157.861 107.746) (width 0.25) (layer B.Cu) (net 22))
 (segment (start 157.861 107.746) (end 157.861 103.1826) (width 0.25) (layer B.Cu) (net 22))
 (segment (start 157.861 103.1826) (end 158.264 102.7796) (width 0.25) (layer B.Cu) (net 22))
 (segment (start 160.044 96.9543) (end 160.044 102.7796) (width 0.25) (layer B.Cu) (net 23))
 (segment (start 156.591 109.855) (end 157.7663 109.855) (width 0.25) (layer B.Cu) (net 23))
 (segment (start 157.7663 109.855) (end 157.7663 109.4876) (width 0.25) (layer B.Cu) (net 23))
 (segment (start 157.7663 109.4876) (end 158.5742 108.6797) (width 0.25) (layer B.Cu) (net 23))
 (segment (start 158.5742 108.6797) (end 159.4673 108.6797) (width 0.25) (layer B.Cu) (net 23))
 (segment (start 159.4673 108.6797) (end 160.3117 107.8353) (width 0.25) (layer B.Cu) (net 23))
 (segment (start 160.3117 107.8353) (end 160.3117 103.0473) (width 0.25) (layer B.Cu) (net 23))
 (segment (start 160.3117 103.0473) (end 160.044 102.7796) (width 0.25) (layer B.Cu) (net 23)))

